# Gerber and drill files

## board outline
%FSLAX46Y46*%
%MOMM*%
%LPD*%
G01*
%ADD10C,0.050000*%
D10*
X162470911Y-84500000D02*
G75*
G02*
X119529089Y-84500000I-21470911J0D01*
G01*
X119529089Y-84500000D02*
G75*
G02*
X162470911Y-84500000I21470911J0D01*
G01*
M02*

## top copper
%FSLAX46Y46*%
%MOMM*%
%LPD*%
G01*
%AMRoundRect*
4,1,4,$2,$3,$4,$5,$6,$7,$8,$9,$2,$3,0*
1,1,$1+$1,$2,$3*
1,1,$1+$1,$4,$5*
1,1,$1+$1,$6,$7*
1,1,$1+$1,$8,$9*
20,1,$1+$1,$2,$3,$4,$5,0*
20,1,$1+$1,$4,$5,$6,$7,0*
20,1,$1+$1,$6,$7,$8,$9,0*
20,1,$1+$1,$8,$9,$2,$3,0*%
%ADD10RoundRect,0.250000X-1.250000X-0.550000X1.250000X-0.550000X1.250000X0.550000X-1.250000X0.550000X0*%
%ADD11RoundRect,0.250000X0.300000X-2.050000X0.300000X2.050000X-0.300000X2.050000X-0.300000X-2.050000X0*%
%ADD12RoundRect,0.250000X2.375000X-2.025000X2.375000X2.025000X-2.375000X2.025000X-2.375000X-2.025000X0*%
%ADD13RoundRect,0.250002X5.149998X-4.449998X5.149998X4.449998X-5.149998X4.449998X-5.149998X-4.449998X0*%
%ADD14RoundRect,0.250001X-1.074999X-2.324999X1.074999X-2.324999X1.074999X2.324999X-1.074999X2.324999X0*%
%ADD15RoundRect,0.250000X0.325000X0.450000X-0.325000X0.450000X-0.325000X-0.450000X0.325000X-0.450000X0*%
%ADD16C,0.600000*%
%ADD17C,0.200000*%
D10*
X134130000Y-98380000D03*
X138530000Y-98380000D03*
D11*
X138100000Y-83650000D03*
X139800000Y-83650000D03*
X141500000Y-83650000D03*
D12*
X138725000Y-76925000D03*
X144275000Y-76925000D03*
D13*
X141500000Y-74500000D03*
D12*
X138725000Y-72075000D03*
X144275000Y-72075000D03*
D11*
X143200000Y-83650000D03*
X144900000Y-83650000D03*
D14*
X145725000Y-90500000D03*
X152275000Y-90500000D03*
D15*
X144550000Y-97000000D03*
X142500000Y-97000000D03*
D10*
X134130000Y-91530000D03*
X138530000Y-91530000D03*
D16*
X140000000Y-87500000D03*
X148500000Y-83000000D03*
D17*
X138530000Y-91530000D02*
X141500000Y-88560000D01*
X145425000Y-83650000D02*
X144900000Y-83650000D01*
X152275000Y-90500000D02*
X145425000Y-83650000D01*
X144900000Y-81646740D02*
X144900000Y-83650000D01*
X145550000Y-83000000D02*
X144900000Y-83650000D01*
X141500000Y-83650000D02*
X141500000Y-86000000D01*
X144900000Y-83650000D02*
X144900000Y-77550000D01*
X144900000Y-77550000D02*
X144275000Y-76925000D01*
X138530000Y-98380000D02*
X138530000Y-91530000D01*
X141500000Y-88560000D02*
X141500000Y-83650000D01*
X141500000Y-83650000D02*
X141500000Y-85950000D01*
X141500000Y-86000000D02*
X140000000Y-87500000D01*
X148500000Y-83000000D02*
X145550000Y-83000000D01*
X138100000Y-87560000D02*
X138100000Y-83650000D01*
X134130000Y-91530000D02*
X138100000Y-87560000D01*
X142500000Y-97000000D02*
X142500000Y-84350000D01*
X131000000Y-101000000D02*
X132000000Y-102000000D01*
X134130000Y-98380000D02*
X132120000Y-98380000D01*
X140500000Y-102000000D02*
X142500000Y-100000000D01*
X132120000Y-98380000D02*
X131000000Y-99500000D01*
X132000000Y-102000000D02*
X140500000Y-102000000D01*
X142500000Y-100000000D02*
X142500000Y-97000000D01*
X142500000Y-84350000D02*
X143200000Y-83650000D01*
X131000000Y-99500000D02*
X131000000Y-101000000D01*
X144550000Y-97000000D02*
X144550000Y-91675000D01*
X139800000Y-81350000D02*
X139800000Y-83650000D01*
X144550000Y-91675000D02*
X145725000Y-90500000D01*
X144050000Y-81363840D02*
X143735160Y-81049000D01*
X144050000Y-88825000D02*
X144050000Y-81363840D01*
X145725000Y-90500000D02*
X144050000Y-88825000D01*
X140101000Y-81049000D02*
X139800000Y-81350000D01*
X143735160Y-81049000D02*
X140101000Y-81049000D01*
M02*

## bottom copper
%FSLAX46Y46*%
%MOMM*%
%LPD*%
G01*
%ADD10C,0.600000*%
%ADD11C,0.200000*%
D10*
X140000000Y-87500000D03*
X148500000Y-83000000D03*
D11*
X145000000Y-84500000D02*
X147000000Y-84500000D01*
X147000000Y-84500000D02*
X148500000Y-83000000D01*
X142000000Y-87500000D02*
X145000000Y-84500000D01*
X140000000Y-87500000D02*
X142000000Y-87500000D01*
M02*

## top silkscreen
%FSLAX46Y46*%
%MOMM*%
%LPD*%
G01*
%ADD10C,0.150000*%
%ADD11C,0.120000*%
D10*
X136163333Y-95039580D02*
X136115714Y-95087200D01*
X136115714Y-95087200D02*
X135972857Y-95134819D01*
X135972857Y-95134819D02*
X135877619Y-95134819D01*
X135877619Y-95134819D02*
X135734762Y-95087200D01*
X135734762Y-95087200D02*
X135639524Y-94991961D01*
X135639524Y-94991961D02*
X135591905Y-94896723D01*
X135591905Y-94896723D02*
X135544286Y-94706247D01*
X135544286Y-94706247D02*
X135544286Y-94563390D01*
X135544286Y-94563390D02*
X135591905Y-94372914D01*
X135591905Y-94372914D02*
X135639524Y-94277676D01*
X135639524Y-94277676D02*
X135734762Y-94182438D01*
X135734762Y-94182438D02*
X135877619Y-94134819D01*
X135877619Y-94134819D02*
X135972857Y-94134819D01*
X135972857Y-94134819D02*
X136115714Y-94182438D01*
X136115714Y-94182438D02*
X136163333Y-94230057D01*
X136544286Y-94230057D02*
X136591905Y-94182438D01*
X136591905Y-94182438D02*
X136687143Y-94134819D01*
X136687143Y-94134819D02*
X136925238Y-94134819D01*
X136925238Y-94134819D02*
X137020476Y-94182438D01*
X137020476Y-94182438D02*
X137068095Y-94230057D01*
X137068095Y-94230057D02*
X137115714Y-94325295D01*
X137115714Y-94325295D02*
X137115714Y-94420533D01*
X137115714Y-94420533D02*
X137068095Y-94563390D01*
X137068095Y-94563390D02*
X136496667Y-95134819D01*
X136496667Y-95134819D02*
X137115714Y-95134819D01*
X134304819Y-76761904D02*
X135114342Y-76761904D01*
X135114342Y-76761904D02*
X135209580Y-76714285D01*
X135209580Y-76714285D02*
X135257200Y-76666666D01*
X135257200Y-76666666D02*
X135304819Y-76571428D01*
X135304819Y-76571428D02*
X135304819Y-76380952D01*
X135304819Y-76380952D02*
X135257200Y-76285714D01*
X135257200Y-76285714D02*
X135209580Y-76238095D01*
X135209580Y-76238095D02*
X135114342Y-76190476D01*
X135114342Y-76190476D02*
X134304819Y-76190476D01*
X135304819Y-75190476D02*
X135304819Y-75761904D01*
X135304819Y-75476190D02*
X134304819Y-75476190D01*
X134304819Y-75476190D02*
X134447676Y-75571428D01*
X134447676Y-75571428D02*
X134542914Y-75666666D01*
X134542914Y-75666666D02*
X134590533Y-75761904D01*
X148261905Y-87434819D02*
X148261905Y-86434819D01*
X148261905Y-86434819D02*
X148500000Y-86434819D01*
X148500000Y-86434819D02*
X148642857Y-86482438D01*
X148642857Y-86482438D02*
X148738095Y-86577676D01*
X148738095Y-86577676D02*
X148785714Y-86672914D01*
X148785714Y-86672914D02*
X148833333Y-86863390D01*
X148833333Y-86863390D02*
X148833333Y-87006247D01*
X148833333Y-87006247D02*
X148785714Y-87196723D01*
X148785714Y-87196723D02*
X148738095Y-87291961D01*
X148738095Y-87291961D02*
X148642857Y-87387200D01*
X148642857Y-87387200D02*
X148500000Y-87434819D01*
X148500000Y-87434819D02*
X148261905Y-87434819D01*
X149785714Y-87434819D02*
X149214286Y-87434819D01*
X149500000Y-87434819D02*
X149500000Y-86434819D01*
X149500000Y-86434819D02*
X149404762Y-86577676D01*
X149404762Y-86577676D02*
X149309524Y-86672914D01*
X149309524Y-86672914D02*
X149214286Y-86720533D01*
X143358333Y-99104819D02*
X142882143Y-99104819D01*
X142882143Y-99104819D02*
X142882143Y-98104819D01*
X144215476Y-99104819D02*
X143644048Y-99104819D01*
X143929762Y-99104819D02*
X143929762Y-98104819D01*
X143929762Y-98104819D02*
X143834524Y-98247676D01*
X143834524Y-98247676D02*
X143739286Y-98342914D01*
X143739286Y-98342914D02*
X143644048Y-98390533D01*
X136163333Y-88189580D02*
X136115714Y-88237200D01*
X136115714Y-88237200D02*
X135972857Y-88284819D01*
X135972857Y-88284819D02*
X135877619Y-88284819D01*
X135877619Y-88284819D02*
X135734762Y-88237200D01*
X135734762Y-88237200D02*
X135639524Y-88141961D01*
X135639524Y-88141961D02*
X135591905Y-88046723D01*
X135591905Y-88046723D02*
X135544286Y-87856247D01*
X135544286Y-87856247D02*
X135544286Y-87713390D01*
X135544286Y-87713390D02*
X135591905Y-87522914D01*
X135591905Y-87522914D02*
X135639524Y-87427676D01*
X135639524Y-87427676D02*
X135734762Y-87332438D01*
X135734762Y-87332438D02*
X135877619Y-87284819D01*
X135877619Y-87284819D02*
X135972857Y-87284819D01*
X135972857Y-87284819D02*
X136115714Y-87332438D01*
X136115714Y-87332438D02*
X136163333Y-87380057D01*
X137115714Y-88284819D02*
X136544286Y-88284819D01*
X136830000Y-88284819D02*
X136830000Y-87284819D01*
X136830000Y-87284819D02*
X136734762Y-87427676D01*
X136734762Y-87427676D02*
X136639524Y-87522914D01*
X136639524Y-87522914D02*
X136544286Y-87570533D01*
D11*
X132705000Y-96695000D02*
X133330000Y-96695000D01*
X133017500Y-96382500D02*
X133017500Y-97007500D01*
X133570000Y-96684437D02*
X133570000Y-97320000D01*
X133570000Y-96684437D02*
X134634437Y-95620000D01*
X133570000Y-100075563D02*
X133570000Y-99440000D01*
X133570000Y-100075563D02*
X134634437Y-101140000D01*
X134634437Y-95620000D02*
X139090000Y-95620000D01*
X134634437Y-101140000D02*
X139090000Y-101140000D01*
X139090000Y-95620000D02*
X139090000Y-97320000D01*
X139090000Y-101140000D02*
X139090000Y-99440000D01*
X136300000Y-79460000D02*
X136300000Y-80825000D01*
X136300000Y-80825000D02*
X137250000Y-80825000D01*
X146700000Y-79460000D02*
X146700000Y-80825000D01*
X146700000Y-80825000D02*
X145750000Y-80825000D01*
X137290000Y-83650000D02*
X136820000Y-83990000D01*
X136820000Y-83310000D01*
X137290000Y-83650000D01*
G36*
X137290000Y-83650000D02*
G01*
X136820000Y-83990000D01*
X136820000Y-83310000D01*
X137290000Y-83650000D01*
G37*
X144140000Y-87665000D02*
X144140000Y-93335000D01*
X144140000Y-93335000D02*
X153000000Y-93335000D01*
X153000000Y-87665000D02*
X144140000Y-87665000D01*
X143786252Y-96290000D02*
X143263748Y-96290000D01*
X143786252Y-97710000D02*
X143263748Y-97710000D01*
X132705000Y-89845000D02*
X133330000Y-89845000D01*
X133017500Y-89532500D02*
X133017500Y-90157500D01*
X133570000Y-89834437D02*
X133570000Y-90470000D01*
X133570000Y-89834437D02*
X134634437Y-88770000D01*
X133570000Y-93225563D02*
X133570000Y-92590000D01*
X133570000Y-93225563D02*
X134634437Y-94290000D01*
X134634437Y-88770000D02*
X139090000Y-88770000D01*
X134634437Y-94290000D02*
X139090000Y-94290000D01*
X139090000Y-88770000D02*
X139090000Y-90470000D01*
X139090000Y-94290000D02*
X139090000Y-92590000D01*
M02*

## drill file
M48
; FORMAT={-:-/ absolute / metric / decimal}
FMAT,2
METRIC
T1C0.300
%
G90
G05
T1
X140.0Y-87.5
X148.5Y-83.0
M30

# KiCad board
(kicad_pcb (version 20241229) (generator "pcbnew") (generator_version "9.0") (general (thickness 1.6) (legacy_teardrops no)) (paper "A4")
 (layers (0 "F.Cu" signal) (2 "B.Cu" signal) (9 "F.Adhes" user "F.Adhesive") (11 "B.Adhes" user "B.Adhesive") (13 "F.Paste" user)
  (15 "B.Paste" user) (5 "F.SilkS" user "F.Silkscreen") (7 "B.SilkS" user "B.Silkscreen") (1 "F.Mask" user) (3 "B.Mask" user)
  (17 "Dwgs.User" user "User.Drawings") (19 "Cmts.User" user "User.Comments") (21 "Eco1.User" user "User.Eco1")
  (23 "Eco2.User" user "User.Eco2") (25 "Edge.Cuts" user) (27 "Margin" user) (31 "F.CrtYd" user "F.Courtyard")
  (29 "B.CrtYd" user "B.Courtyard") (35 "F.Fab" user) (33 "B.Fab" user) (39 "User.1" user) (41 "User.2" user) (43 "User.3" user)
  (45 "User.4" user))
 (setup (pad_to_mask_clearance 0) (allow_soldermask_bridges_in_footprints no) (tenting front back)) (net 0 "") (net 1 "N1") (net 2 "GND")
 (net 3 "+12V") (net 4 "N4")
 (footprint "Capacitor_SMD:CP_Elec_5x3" (layer "F.Cu") (at 136.33 98.38)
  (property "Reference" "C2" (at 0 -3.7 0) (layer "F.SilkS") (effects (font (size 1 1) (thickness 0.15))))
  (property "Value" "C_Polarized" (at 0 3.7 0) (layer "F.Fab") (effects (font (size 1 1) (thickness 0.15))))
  (fp_line (start -3.625 -1.685) (end -3 -1.685) (stroke (width 0.12) (type solid)) (layer "F.SilkS"))
  (fp_line (start -3.3125 -1.9975) (end -3.3125 -1.3725) (stroke (width 0.12) (type solid)) (layer "F.SilkS"))
  (fp_line (start -2.76 -1.695563) (end -2.76 -1.06) (stroke (width 0.12) (type solid)) (layer "F.SilkS"))
  (fp_line (start -2.76 -1.695563) (end -1.695563 -2.76) (stroke (width 0.12) (type solid)) (layer "F.SilkS"))
  (fp_line (start -2.76 1.695563) (end -2.76 1.06) (stroke (width 0.12) (type solid)) (layer "F.SilkS"))
  (fp_line (start -2.76 1.695563) (end -1.695563 2.76) (stroke (width 0.12) (type solid)) (layer "F.SilkS"))
  (fp_line (start -1.695563 -2.76) (end 2.76 -2.76) (stroke (width 0.12) (type solid)) (layer "F.SilkS"))
  (fp_line (start -1.695563 2.76) (end 2.76 2.76) (stroke (width 0.12) (type solid)) (layer "F.SilkS"))
  (fp_line (start 2.76 -2.76) (end 2.76 -1.06) (stroke (width 0.12) (type solid)) (layer "F.SilkS"))
  (fp_line (start 2.76 2.76) (end 2.76 1.06) (stroke (width 0.12) (type solid)) (layer "F.SilkS"))
  (pad "1" smd roundrect (at -2.2 0) (size 3 1.6) (layers "F.Cu" "F.Mask" "F.Paste") (roundrect_rratio 0.15625) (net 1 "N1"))
  (pad "2" smd roundrect (at 2.2 0) (size 3 1.6) (layers "F.Cu" "F.Mask" "F.Paste") (roundrect_rratio 0.15625) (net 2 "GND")))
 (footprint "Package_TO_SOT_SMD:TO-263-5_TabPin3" (layer "F.Cu") (at 141.5 76 90)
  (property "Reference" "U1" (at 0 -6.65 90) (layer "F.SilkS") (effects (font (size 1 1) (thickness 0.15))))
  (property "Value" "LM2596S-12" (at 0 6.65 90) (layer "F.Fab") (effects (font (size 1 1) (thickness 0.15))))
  (fp_line (start -3.46 -5.2) (end -4.825 -5.2) (stroke (width 0.12) (type solid)) (layer "F.SilkS"))
  (fp_line (start -4.825 -5.2) (end -4.825 -4.25) (stroke (width 0.12) (type solid)) (layer "F.SilkS"))
  (fp_line (start -3.46 5.2) (end -4.825 5.2) (stroke (width 0.12) (type solid)) (layer "F.SilkS"))
  (fp_line (start -4.825 5.2) (end -4.825 4.25) (stroke (width 0.12) (type solid)) (layer "F.SilkS"))
  (fp_poly
   (pts (xy -7.65 -4.21) (xy -7.99 -4.68) (xy -7.31 -4.68) (xy -7.65 -4.21)) (stroke (width 0.12) (type solid)) (fill yes) (layer "F.SilkS"))
  (pad "1" smd roundrect (at -7.65 -3.4 90) (size 4.6 1.1) (layers "F.Cu" "F.Mask" "F.Paste") (roundrect_rratio 0.227273) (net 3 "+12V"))
  (pad "2" smd roundrect (at -7.65 -1.7 90) (size 4.6 1.1) (layers "F.Cu" "F.Mask" "F.Paste") (roundrect_rratio 0.227273) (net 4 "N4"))
  (pad "3" smd roundrect (at -7.65 0 90) (size 4.6 1.1) (layers "F.Cu" "F.Mask" "F.Paste") (roundrect_rratio 0.227273) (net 2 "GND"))
  (pad "3" smd roundrect (at -0.925 -2.775 90) (size 4.55 5.25) (layers "F.Cu" "F.Paste") (roundrect_rratio 0.054945) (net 2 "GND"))
  (pad "3" smd roundrect (at -0.925 2.775 90) (size 4.55 5.25) (layers "F.Cu" "F.Paste") (roundrect_rratio 0.054945) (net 2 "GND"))
  (pad "3" smd roundrect (at 1.5 0 90) (size 9.4 10.8) (layers "F.Cu" "F.Mask") (roundrect_rratio 0.026596) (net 2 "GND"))
  (pad "3" smd roundrect (at 3.925 -2.775 90) (size 4.55 5.25) (layers "F.Cu" "F.Paste") (roundrect_rratio 0.054945) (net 2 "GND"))
  (pad "3" smd roundrect (at 3.925 2.775 90) (size 4.55 5.25) (layers "F.Cu" "F.Paste") (roundrect_rratio 0.054945) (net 2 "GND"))
  (pad "4" smd roundrect (at -7.65 1.7 90) (size 4.6 1.1) (layers "F.Cu" "F.Mask" "F.Paste") (roundrect_rratio 0.227273) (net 1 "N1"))
  (pad "5" smd roundrect (at -7.65 3.4 90) (size 4.6 1.1) (layers "F.Cu" "F.Mask" "F.Paste") (roundrect_rratio 0.227273) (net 2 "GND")))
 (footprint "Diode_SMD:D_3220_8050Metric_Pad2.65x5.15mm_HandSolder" (layer "F.Cu") (at 149 90.5)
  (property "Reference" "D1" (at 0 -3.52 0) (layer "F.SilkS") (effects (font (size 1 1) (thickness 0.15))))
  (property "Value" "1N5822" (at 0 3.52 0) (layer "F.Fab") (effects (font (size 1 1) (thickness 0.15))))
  (fp_line (start -4.86 -2.835) (end -4.86 2.835) (stroke (width 0.12) (type solid)) (layer "F.SilkS"))
  (fp_line (start -4.86 2.835) (end 4 2.835) (stroke (width 0.12) (type solid)) (layer "F.SilkS"))
  (fp_line (start 4 -2.835) (end -4.86 -2.835) (stroke (width 0.12) (type solid)) (layer "F.SilkS"))
  (pad "1" smd roundrect (at -3.275 0) (size 2.65 5.15) (layers "F.Cu" "F.Mask" "F.Paste") (roundrect_rratio 0.09434) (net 4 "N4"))
  (pad "2" smd roundrect (at 3.275 0) (size 2.65 5.15) (layers "F.Cu" "F.Mask" "F.Paste") (roundrect_rratio 0.09434) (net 2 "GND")))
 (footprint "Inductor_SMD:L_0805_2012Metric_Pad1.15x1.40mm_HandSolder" (layer "F.Cu") (at 143.525 97 180)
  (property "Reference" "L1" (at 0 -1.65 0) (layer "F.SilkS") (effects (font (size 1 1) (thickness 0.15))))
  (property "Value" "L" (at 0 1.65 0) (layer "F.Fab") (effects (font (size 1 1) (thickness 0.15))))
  (fp_line (start -0.261252 0.71) (end 0.261252 0.71) (stroke (width 0.12) (type solid)) (layer "F.SilkS"))
  (fp_line (start -0.261252 -0.71) (end 0.261252 -0.71) (stroke (width 0.12) (type solid)) (layer "F.SilkS"))
  (pad "1" smd roundrect (at -1.025 0 180) (size 1.15 1.4) (layers "F.Cu" "F.Mask" "F.Paste") (roundrect_rratio 0.217391) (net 4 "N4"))
  (pad "2" smd roundrect (at 1.025 0 180) (size 1.15 1.4) (layers "F.Cu" "F.Mask" "F.Paste") (roundrect_rratio 0.217391) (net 1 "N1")))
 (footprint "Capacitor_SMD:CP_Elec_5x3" (layer "F.Cu") (at 136.33 91.53)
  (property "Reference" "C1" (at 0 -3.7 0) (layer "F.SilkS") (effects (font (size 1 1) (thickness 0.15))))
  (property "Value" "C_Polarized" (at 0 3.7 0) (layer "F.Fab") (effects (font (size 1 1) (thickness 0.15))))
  (fp_line (start -3.625 -1.685) (end -3 -1.685) (stroke (width 0.12) (type solid)) (layer "F.SilkS"))
  (fp_line (start -3.3125 -1.9975) (end -3.3125 -1.3725) (stroke (width 0.12) (type solid)) (layer "F.SilkS"))
  (fp_line (start -2.76 -1.695563) (end -2.76 -1.06) (stroke (width 0.12) (type solid)) (layer "F.SilkS"))
  (fp_line (start -2.76 -1.695563) (end -1.695563 -2.76) (stroke (width 0.12) (type solid)) (layer "F.SilkS"))
  (fp_line (start -2.76 1.695563) (end -2.76 1.06) (stroke (width 0.12) (type solid)) (layer "F.SilkS"))
  (fp_line (start -2.76 1.695563) (end -1.695563 2.76) (stroke (width 0.12) (type solid)) (layer "F.SilkS"))
  (fp_line (start -1.695563 -2.76) (end 2.76 -2.76) (stroke (width 0.12) (type solid)) (layer "F.SilkS"))
  (fp_line (start -1.695563 2.76) (end 2.76 2.76) (stroke (width 0.12) (type solid)) (layer "F.SilkS"))
  (fp_line (start 2.76 -2.76) (end 2.76 -1.06) (stroke (width 0.12) (type solid)) (layer "F.SilkS"))
  (fp_line (start 2.76 2.76) (end 2.76 1.06) (stroke (width 0.12) (type solid)) (layer "F.SilkS"))
  (pad "1" smd roundrect (at -2.2 0) (size 3 1.6) (layers "F.Cu" "F.Mask" "F.Paste") (roundrect_rratio 0.15625) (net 3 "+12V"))
  (pad "2" smd roundrect (at 2.2 0) (size 3 1.6) (layers "F.Cu" "F.Mask" "F.Paste") (roundrect_rratio 0.15625) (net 2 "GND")))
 (gr_circle (center 141 84.5) (end 160 94.5) (stroke (width 0.05) (type default)) (fill no) (layer "Edge.Cuts"))
 (segment (start 138.53 91.53) (end 141.5 88.56) (width 0.2) (layer "F.Cu") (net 2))
 (segment (start 145.425 83.65) (end 144.9 83.65) (width 0.2) (layer "F.Cu") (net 2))
 (segment (start 152.275 90.5) (end 145.425 83.65) (width 0.2) (layer "F.Cu") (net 2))
 (segment (start 144.9 81.64674) (end 144.9 83.65) (width 0.2) (layer "F.Cu") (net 2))
 (segment (start 145.55 83) (end 144.9 83.65) (width 0.2) (layer "F.Cu") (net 2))
 (segment (start 141.5 83.65) (end 141.5 86) (width 0.2) (layer "F.Cu") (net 2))
 (segment (start 144.9 83.65) (end 144.9 77.55) (width 0.2) (layer "F.Cu") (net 2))
 (segment (start 144.9 77.55) (end 144.275 76.925) (width 0.2) (layer "F.Cu") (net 2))
 (segment (start 138.53 98.38) (end 138.53 91.53) (width 0.2) (layer "F.Cu") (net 2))
 (segment (start 141.5 88.56) (end 141.5 83.65) (width 0.2) (layer "F.Cu") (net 2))
 (segment (start 141.5 83.65) (end 141.5 85.95) (width 0.2) (layer "F.Cu") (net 2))
 (segment (start 141.5 86) (end 140 87.5) (width 0.2) (layer "F.Cu") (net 2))
 (segment (start 148.5 83) (end 145.55 83) (width 0.2) (layer "F.Cu") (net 2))
 (via (at 140 87.5) (size 0.6) (drill 0.3) (layers "F.Cu" "B.Cu") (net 2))
 (via (at 148.5 83) (size 0.6) (drill 0.3) (layers "F.Cu" "B.Cu") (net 2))
 (segment (start 145 84.5) (end 147 84.5) (width 0.2) (layer "B.Cu") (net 2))
 (segment (start 147 84.5) (end 148.5 83) (width 0.2) (layer "B.Cu") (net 2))
 (segment (start 142 87.5) (end 145 84.5) (width 0.2) (layer "B.Cu") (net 2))
 (segment (start 140 87.5) (end 142 87.5) (width 0.2) (layer "B.Cu") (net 2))
 (segment (start 138.1 87.56) (end 138.1 83.65) (width 0.2) (layer "F.Cu") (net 3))
 (segment (start 134.13 91.53) (end 138.1 87.56) (width 0.2) (layer "F.Cu") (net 3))
 (segment (start 142.5 97) (end 142.5 84.35) (width 0.2) (layer "F.Cu") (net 1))
 (segment (start 131 101) (end 132 102) (width 0.2) (layer "F.Cu") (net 1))
 (segment (start 134.13 98.38) (end 132.12 98.38) (width 0.2) (layer "F.Cu") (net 1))
 (segment (start 140.5 102) (end 142.5 100) (width 0.2) (layer "F.Cu") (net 1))
 (segment (start 132.12 98.38) (end 131 99.5) (width 0.2) (layer "F.Cu") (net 1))
 (segment (start 132 102) (end 140.5 102) (width 0.2) (layer "F.Cu") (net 1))
 (segment (start 142.5 100) (end 142.5 97) (width 0.2) (layer "F.Cu") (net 1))
 (segment (start 142.5 84.35) (end 143.2 83.65) (width 0.2) (layer "F.Cu") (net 1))
 (segment (start 131 99.5) (end 131 101) (width 0.2) (layer "F.Cu") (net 1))
 (segment (start 144.55 97) (end 144.55 91.675) (width 0.2) (layer "F.Cu") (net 4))
 (segment (start 139.8 81.35) (end 139.8 83.65) (width 0.2) (layer "F.Cu") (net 4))
 (segment (start 144.55 91.675) (end 145.725 90.5) (width 0.2) (layer "F.Cu") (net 4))
 (segment (start 144.05 81.36384) (end 143.73516 81.049) (width 0.2) (layer "F.Cu") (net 4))
 (segment (start 144.05 88.825) (end 144.05 81.36384) (width 0.2) (layer "F.Cu") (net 4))
 (segment (start 145.725 90.5) (end 144.05 88.825) (width 0.2) (layer "F.Cu") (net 4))
 (segment (start 140.101 81.049) (end 139.8 81.35) (width 0.2) (layer "F.Cu") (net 4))
 (segment (start 143.73516 81.049) (end 140.101 81.049) (width 0.2) (layer "F.Cu") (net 4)))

